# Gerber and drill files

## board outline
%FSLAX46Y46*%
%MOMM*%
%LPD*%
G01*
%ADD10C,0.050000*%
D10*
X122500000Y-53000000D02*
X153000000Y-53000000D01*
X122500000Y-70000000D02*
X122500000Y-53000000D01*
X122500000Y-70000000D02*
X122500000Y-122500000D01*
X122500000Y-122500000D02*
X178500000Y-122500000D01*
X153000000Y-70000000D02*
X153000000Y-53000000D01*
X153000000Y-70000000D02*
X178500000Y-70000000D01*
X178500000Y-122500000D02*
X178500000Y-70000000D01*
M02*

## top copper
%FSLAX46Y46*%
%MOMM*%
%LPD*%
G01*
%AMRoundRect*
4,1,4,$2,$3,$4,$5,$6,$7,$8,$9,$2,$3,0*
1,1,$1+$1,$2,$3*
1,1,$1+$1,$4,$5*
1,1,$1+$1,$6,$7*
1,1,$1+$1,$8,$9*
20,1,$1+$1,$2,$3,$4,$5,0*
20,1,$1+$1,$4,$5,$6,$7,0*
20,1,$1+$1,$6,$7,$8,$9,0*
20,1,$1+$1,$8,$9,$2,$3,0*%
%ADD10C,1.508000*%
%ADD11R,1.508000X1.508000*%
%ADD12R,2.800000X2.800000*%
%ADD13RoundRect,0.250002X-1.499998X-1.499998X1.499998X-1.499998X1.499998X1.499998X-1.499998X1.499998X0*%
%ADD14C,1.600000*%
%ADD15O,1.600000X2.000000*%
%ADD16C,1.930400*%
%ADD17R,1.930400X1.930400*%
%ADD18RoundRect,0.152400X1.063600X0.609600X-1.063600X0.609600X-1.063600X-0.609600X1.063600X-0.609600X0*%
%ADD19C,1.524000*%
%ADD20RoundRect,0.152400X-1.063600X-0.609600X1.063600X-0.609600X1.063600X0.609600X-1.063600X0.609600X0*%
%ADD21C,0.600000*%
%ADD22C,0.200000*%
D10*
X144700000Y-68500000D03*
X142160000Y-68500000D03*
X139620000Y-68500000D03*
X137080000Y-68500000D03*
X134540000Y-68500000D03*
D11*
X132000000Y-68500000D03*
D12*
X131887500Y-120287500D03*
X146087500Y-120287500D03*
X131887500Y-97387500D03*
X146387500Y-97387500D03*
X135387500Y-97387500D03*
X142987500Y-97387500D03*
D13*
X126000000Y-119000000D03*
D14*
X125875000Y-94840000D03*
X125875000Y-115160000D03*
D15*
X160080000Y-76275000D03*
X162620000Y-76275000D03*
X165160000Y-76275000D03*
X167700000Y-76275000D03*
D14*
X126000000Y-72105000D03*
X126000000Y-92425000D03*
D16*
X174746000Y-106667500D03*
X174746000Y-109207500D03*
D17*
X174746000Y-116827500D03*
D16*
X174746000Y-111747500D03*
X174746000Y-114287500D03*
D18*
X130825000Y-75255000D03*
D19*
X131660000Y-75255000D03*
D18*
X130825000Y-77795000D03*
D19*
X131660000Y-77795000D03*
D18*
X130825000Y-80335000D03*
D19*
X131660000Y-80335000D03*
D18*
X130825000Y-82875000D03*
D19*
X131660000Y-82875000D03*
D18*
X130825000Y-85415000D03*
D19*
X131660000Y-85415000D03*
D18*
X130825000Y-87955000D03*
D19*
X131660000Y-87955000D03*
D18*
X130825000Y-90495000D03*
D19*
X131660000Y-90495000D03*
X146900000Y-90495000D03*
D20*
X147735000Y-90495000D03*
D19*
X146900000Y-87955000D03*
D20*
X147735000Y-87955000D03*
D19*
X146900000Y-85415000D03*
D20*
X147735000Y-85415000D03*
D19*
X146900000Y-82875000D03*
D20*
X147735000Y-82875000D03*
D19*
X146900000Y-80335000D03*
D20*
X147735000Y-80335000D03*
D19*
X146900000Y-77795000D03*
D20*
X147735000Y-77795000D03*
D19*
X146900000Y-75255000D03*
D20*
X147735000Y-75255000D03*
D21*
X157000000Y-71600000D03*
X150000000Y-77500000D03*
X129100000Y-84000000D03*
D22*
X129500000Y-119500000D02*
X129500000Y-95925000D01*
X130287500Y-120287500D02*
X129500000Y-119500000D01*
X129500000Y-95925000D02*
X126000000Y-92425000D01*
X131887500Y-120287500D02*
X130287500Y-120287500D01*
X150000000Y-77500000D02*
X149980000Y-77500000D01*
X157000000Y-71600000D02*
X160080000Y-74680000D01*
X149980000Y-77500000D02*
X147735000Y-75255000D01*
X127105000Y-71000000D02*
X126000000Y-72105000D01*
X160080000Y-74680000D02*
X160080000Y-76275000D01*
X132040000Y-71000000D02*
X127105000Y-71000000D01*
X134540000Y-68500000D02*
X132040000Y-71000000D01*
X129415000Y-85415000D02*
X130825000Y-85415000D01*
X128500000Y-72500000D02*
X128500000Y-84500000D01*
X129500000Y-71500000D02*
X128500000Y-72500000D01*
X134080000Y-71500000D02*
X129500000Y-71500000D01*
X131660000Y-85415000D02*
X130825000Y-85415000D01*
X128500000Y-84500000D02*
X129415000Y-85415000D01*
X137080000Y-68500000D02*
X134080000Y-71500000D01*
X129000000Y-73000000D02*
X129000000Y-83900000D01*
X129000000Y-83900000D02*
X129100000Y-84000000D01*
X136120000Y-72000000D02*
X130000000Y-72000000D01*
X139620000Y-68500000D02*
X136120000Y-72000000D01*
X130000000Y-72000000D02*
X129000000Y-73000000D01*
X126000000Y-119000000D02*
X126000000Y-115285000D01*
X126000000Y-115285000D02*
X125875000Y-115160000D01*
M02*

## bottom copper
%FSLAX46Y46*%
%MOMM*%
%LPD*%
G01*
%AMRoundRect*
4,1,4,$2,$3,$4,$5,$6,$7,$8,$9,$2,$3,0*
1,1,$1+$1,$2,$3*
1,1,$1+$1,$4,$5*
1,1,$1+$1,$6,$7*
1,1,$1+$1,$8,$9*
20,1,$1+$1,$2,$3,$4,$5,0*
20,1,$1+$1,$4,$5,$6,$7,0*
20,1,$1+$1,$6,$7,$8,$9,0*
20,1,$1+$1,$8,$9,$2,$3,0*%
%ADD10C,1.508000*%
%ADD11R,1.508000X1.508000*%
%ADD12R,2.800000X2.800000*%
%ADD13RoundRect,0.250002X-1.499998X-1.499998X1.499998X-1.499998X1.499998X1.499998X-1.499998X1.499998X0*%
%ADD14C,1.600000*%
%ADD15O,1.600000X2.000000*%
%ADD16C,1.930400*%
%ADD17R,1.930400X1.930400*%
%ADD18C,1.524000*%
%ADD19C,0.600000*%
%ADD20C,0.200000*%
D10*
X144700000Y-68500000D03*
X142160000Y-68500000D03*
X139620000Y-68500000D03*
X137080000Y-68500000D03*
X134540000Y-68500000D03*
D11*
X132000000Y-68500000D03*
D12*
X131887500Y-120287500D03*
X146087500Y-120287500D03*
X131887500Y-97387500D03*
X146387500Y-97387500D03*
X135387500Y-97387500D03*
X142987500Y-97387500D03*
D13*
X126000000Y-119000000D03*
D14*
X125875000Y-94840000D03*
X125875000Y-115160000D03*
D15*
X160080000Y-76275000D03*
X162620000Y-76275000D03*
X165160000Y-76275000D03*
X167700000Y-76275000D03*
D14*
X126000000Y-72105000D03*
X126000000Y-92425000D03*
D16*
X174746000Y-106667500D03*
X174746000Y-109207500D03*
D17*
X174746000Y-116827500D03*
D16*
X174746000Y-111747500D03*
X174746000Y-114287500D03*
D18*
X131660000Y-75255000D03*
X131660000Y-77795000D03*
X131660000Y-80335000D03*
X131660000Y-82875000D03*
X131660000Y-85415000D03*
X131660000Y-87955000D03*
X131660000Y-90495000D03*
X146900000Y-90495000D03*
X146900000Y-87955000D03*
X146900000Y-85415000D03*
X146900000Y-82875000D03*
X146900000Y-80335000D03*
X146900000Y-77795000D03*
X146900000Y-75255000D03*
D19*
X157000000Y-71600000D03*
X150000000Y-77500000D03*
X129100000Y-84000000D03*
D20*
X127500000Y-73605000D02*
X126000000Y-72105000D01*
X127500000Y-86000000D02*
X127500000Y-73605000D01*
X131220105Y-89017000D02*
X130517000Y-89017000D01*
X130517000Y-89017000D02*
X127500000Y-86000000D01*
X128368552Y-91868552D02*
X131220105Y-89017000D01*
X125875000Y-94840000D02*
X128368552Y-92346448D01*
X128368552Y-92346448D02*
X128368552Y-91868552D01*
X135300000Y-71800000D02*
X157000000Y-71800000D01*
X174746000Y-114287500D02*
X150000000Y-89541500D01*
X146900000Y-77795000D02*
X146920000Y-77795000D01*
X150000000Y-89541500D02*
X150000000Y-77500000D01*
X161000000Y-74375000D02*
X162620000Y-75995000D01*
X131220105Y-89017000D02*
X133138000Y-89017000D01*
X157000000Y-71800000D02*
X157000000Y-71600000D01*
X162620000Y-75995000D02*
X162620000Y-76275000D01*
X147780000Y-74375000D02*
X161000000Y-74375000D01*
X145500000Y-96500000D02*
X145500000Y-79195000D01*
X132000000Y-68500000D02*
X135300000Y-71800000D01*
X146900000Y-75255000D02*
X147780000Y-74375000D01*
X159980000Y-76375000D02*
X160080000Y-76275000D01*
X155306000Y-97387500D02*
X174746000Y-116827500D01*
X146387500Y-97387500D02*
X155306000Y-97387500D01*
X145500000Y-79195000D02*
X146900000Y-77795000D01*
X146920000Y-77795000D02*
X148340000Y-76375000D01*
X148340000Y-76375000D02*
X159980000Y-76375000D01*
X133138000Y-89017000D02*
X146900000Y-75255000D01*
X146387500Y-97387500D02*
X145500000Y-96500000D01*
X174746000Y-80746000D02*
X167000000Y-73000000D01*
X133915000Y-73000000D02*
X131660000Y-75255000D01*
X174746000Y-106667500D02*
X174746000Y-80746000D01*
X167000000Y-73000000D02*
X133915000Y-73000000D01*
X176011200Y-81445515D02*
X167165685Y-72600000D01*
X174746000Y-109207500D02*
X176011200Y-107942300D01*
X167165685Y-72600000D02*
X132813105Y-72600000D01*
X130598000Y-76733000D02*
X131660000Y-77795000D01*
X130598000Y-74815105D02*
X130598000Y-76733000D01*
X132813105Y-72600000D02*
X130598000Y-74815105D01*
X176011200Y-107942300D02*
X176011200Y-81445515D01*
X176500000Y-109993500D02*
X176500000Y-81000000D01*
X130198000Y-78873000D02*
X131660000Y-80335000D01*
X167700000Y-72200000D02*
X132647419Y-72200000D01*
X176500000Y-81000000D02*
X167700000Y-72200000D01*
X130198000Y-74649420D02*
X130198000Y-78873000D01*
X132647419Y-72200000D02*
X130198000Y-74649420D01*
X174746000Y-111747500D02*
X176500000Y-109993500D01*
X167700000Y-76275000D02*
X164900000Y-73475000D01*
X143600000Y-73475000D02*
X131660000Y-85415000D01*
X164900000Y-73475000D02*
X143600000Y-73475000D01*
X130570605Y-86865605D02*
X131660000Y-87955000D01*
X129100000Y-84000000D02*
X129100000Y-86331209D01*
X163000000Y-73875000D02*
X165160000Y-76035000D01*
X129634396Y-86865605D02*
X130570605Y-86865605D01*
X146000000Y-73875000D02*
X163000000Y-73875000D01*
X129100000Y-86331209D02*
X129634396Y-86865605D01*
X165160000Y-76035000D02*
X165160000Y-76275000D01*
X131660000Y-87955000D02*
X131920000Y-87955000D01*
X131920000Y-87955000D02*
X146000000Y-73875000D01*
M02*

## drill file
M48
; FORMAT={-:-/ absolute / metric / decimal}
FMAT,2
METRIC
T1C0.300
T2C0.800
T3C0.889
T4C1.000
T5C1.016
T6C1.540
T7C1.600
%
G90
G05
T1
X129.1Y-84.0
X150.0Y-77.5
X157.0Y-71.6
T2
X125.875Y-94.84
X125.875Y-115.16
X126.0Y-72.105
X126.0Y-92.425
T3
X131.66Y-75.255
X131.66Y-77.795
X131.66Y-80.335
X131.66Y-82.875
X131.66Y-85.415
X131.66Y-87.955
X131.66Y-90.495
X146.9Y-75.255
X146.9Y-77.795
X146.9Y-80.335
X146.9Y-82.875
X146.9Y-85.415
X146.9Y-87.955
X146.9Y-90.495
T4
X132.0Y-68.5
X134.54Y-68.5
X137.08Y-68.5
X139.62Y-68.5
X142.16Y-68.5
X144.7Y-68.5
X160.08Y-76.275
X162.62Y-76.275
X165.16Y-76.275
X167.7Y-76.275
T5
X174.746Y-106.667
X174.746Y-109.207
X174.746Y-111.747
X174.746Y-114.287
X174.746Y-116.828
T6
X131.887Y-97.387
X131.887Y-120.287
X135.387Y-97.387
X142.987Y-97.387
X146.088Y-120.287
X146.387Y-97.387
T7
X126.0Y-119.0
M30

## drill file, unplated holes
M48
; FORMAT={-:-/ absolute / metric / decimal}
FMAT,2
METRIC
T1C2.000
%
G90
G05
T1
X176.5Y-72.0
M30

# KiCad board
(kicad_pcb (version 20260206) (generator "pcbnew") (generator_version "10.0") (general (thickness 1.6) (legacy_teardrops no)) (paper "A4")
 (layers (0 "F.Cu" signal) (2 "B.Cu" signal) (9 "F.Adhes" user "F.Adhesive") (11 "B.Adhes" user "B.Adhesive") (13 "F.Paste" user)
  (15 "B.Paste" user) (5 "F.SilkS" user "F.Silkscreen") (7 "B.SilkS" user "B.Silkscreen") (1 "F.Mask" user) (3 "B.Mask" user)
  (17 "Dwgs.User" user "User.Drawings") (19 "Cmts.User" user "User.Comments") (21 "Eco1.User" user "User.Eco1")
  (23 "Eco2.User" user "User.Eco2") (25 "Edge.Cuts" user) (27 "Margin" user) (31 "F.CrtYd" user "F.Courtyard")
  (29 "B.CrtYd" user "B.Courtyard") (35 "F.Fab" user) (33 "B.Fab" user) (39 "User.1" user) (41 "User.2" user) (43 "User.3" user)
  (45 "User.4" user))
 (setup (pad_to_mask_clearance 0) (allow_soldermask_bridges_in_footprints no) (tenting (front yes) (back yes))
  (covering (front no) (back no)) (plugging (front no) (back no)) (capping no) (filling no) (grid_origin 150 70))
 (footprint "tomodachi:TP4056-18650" (layer "F.Cu") (at 130.1875 121.9875 90)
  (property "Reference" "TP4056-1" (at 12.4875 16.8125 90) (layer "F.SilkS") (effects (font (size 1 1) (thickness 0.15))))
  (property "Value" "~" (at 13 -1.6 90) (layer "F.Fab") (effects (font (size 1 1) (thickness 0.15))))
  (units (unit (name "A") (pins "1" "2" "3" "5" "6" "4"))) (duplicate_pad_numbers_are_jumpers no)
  (pad "1" thru_hole rect (at 1.7 1.7 90) (size 2.8 2.8) (drill 1.54) (layers "*.Cu" "*.Mask") (remove_unused_layers no) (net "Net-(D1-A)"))
  (pad "2" thru_hole rect (at 1.7 15.9 90) (size 2.8 2.8) (drill 1.54) (layers "*.Cu" "*.Mask") (remove_unused_layers no) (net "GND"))
  (pad "3" thru_hole rect (at 24.6 1.7 90) (size 2.8 2.8) (drill 1.54) (layers "*.Cu" "*.Mask") (remove_unused_layers no)
   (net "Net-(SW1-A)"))
  (pad "4" thru_hole rect (at 24.6 16.2 90) (size 2.8 2.8) (drill 1.54) (layers "*.Cu" "*.Mask") (remove_unused_layers no)
   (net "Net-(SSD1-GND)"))
  (pad "5" thru_hole rect (at 24.6 5.2 90) (size 2.8 2.8) (drill 1.54) (layers "*.Cu" "*.Mask") (remove_unused_layers no)
   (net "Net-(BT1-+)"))
  (pad "6" thru_hole rect (at 24.6 12.8 90) (size 2.8 2.8) (drill 1.54) (layers "*.Cu" "*.Mask") (remove_unused_layers no)
   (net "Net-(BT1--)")))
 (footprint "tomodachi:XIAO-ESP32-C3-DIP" (layer "F.Cu") (at 139.28 82.875 90)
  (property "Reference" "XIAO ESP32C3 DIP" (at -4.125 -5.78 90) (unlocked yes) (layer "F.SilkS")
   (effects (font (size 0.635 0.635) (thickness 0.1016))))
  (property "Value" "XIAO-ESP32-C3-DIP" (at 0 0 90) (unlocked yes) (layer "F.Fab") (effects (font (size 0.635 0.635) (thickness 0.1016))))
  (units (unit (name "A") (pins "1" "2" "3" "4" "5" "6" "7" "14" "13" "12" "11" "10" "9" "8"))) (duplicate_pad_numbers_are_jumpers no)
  (pad "1" smd roundrect (at 7.62 -8.455 180) (size 2.432 1.524) (layers "F.Cu" "F.Mask") (roundrect_rratio 0.1)
   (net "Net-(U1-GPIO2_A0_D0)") (thermal_bridge_angle 45))
  (pad "1" thru_hole circle (at 7.62 -7.62 180) (size 1.524 1.524) (drill 0.889) (layers "*.Cu" "*.Mask") (remove_unused_layers no)
   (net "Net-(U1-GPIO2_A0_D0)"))
  (pad "2" smd roundrect (at 5.08 -8.455 180) (size 2.432 1.524) (layers "F.Cu" "F.Mask") (roundrect_rratio 0.1)
   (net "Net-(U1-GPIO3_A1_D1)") (thermal_bridge_angle 45))
  (pad "2" thru_hole circle (at 5.08 -7.62 180) (size 1.524 1.524) (drill 0.889) (layers "*.Cu" "*.Mask") (remove_unused_layers no)
   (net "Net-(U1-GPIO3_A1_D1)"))
  (pad "3" smd roundrect (at 2.54 -8.455 180) (size 2.432 1.524) (layers "F.Cu" "F.Mask") (roundrect_rratio 0.1)
   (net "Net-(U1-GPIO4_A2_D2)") (thermal_bridge_angle 45))
  (pad "3" thru_hole circle (at 2.54 -7.62 180) (size 1.524 1.524) (drill 0.889) (layers "*.Cu" "*.Mask") (remove_unused_layers no)
   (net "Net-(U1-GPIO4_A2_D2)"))
  (pad "4" smd roundrect (at 0 -8.455 180) (size 2.432 1.524) (layers "F.Cu" "F.Mask") (roundrect_rratio 0.1)
   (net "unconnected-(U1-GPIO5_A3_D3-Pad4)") (thermal_bridge_angle 45))
  (pad "4" thru_hole circle (at 0 -7.62 180) (size 1.524 1.524) (drill 0.889) (layers "*.Cu" "*.Mask") (remove_unused_layers no)
   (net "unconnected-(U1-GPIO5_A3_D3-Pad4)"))
  (pad "5" smd roundrect (at -2.54 -8.455 180) (size 2.432 1.524) (layers "F.Cu" "F.Mask") (roundrect_rratio 0.1) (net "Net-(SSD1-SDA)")
   (thermal_bridge_angle 45))
  (pad "5" thru_hole circle (at -2.54 -7.62 180) (size 1.524 1.524) (drill 0.889) (layers "*.Cu" "*.Mask") (remove_unused_layers no)
   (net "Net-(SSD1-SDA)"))
  (pad "6" smd roundrect (at -5.08 -8.455 180) (size 2.432 1.524) (layers "F.Cu" "F.Mask") (roundrect_rratio 0.1) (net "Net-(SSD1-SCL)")
   (thermal_bridge_angle 45))
  (pad "6" thru_hole circle (at -5.08 -7.62 180) (size 1.524 1.524) (drill 0.889) (layers "*.Cu" "*.Mask") (remove_unused_layers no)
   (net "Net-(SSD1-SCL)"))
  (pad "7" smd roundrect (at -7.62 -8.455 180) (size 2.432 1.524) (layers "F.Cu" "F.Mask") (roundrect_rratio 0.1)
   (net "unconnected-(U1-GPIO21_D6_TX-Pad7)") (thermal_bridge_angle 45))
  (pad "7" thru_hole circle (at -7.62 -7.62 180) (size 1.524 1.524) (drill 0.889) (layers "*.Cu" "*.Mask") (remove_unused_layers no)
   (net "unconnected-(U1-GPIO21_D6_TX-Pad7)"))
  (pad "8" thru_hole circle (at -7.62 7.62) (size 1.524 1.524) (drill 0.889) (layers "*.Cu" "*.Mask") (remove_unused_layers no)
   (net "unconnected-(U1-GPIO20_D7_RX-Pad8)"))
  (pad "8" smd roundrect (at -7.62 8.455) (size 2.432 1.524) (layers "F.Cu" "F.Mask") (roundrect_rratio 0.1)
   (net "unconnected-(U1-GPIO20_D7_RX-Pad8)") (thermal_bridge_angle 45))
  (pad "9" thru_hole circle (at -5.08 7.62) (size 1.524 1.524) (drill 0.889) (layers "*.Cu" "*.Mask") (remove_unused_layers no)
   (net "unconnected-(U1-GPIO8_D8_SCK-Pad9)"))
  (pad "9" smd roundrect (at -5.08 8.455) (size 2.432 1.524) (layers "F.Cu" "F.Mask") (roundrect_rratio 0.1)
   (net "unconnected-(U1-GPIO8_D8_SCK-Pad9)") (thermal_bridge_angle 45))
  (pad "10" thru_hole circle (at -2.54 7.62) (size 1.524 1.524) (drill 0.889) (layers "*.Cu" "*.Mask") (remove_unused_layers no)
   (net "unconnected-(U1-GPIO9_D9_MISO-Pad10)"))
  (pad "10" smd roundrect (at -2.54 8.455) (size 2.432 1.524) (layers "F.Cu" "F.Mask") (roundrect_rratio 0.1)
   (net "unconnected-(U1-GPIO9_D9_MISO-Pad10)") (thermal_bridge_angle 45))
  (pad "11" thru_hole circle (at 0 7.62) (size 1.524 1.524) (drill 0.889) (layers "*.Cu" "*.Mask") (remove_unused_layers no)
   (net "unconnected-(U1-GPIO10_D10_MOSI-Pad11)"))
  (pad "11" smd roundrect (at 0 8.455) (size 2.432 1.524) (layers "F.Cu" "F.Mask") (roundrect_rratio 0.1)
   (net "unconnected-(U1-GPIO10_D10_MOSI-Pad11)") (thermal_bridge_angle 45))
  (pad "12" thru_hole circle (at 2.54 7.62) (size 1.524 1.524) (drill 0.889) (layers "*.Cu" "*.Mask") (remove_unused_layers no)
   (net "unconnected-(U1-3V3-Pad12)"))
  (pad "12" smd roundrect (at 2.54 8.455) (size 2.432 1.524) (layers "F.Cu" "F.Mask") (roundrect_rratio 0.1)
   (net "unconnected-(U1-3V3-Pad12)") (thermal_bridge_angle 45))
  (pad "13" thru_hole circle (at 5.08 7.62) (size 1.524 1.524) (drill 0.889) (layers "*.Cu" "*.Mask") (remove_unused_layers no)
   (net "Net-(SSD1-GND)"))
  (pad "13" smd roundrect (at 5.08 8.455) (size 2.432 1.524) (layers "F.Cu" "F.Mask") (roundrect_rratio 0.1) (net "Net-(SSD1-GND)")
   (thermal_bridge_angle 45))
  (pad "14" thru_hole circle (at 7.62 7.62) (size 1.524 1.524) (drill 0.889) (layers "*.Cu" "*.Mask") (remove_unused_layers no)
   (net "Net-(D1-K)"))
  (pad "14" smd roundrect (at 7.62 8.455) (size 2.432 1.524) (layers "F.Cu" "F.Mask") (roundrect_rratio 0.1) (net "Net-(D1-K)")
   (thermal_bridge_angle 45)))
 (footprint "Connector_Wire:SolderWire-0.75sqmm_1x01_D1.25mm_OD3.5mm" (layer "F.Cu") (at 126 119)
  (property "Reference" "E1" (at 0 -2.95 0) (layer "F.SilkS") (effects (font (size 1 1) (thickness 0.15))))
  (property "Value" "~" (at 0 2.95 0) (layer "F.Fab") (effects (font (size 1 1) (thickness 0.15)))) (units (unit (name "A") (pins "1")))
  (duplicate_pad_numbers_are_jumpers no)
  (pad "1" thru_hole roundrect (at 0 0) (size 3.5 3.5) (drill 1.6) (layers "*.Cu" "*.Mask") (remove_unused_layers no)
   (roundrect_rratio 0.071429) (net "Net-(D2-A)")))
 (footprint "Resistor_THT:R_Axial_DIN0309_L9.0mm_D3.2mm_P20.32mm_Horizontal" (layer "F.Cu") (at 125.875 94.84 -90)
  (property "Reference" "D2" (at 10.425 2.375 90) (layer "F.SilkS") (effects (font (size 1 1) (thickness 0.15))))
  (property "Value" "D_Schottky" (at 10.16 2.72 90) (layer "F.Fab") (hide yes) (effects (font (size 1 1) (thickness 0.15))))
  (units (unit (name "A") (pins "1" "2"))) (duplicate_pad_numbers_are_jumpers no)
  (pad "1" thru_hole circle (at 0 0 270) (size 1.6 1.6) (drill 0.8) (layers "*.Cu" "*.Mask") (remove_unused_layers no) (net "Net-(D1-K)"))
  (pad "2" thru_hole circle (at 20.32 0 270) (size 1.6 1.6) (drill 0.8) (layers "*.Cu" "*.Mask") (remove_unused_layers no)
   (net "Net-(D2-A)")))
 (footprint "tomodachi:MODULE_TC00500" (layer "F.Cu") (at 138.35 68.5 90)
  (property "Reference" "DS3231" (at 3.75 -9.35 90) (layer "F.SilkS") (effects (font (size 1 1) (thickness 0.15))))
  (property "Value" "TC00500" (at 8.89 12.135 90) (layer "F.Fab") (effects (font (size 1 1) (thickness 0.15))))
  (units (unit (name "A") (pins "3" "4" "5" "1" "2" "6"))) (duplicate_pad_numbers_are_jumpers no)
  (pad "1" thru_hole circle (at 0 6.35 90) (size 1.508 1.508) (drill 1) (layers "*.Cu" "*.Mask") (remove_unused_layers no)
   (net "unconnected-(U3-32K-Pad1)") (solder_mask_margin 0.102))
  (pad "2" thru_hole circle (at 0 3.81 90) (size 1.508 1.508) (drill 1) (layers "*.Cu" "*.Mask") (remove_unused_layers no)
   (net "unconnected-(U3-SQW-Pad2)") (solder_mask_margin 0.102))
  (pad "3" thru_hole circle (at 0 1.27 90) (size 1.508 1.508) (drill 1) (layers "*.Cu" "*.Mask") (remove_unused_layers no)
   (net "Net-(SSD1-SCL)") (solder_mask_margin 0.102))
  (pad "4" thru_hole circle (at 0 -1.27 90) (size 1.508 1.508) (drill 1) (layers "*.Cu" "*.Mask") (remove_unused_layers no)
   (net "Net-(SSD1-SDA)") (solder_mask_margin 0.102))
  (pad "5" thru_hole circle (at 0 -3.81 90) (size 1.508 1.508) (drill 1) (layers "*.Cu" "*.Mask") (remove_unused_layers no)
   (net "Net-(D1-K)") (solder_mask_margin 0.102))
  (pad "6" thru_hole rect (at 0 -6.35 90) (size 1.508 1.508) (drill 1) (layers "*.Cu" "*.Mask") (remove_unused_layers no)
   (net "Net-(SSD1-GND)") (solder_mask_margin 0.102)))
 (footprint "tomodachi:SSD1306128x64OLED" (layer "F.Cu") (at 163.7 86.875)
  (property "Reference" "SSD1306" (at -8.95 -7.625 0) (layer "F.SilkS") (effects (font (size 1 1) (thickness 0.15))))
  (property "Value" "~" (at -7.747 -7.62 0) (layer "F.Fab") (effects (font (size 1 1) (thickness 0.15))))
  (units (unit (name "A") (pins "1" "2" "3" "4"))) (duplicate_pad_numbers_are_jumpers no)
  (pad "1" thru_hole oval (at -3.62 -10.6 90) (size 2 1.6) (drill 1) (layers "*.Cu" "*.Mask") (remove_unused_layers no)
   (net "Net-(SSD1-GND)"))
  (pad "2" thru_hole oval (at -1.08 -10.6 90) (size 2 1.6) (drill 1) (layers "*.Cu" "*.Mask") (remove_unused_layers no) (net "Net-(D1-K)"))
  (pad "3" thru_hole oval (at 1.46 -10.6 90) (size 2 1.6) (drill 1) (layers "*.Cu" "*.Mask") (remove_unused_layers no)
   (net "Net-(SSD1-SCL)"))
  (pad "4" thru_hole oval (at 4 -10.6 90) (size 2 1.6) (drill 1) (layers "*.Cu" "*.Mask") (remove_unused_layers no) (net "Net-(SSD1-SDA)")))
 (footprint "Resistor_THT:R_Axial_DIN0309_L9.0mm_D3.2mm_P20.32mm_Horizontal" (layer "F.Cu") (at 126 72.105 -90)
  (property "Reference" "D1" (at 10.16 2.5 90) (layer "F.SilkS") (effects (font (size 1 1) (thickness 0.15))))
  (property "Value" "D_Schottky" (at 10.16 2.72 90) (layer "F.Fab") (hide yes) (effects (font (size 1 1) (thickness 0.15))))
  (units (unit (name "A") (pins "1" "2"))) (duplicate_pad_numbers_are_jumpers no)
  (pad "1" thru_hole circle (at 0 0 270) (size 1.6 1.6) (drill 0.8) (layers "*.Cu" "*.Mask") (remove_unused_layers no) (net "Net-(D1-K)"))
  (pad "2" thru_hole circle (at 20.32 0 270) (size 1.6 1.6) (drill 0.8) (layers "*.Cu" "*.Mask") (remove_unused_layers no)
   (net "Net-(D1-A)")))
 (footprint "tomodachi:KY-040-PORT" (layer "F.Cu") (at 164 111.875 -90)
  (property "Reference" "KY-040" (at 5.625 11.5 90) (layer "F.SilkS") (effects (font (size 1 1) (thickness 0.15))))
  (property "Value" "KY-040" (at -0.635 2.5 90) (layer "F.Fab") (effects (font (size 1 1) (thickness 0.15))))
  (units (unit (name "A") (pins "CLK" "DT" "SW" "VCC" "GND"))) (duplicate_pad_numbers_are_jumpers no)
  (pad "CLK" thru_hole circle (at -5.2075 -10.746 270) (size 1.9304 1.9304) (drill 1.016) (layers "*.Cu" "*.Mask") (remove_unused_layers no)
   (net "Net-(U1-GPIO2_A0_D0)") (solder_mask_margin 0.102))
  (pad "DT" thru_hole circle (at -2.6675 -10.746 270) (size 1.9304 1.9304) (drill 1.016) (layers "*.Cu" "*.Mask") (remove_unused_layers no)
   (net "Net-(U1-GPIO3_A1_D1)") (solder_mask_margin 0.102))
  (pad "GND" thru_hole rect (at 4.9525 -10.746 270) (size 1.9304 1.9304) (drill 1.016) (layers "*.Cu" "*.Mask") (remove_unused_layers no)
   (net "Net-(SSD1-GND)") (solder_mask_margin 0.102))
  (pad "SW" thru_hole circle (at -0.1275 -10.746 270) (size 1.9304 1.9304) (drill 1.016) (layers "*.Cu" "*.Mask") (remove_unused_layers no)
   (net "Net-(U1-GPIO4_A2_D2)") (solder_mask_margin 0.102))
  (pad "VCC" thru_hole circle (at 2.4125 -10.746 270) (size 1.9304 1.9304) (drill 1.016) (layers "*.Cu" "*.Mask") (remove_unused_layers no)
   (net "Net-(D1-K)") (solder_mask_margin 0.102)))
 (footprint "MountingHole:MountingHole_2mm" (layer "F.Cu") (at 176.5 72)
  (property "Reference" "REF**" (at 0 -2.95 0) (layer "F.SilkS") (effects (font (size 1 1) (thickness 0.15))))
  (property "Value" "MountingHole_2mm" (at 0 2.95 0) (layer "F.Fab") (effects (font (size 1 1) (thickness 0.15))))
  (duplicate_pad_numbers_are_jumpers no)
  (pad "" np_thru_hole circle (at 0 0) (size 2 2) (drill 2) (layers "*.Cu" "*.Mask")))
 (gr_line (start 122.5 53) (end 153 53) (stroke (width 0.05) (type default)) (layer "Edge.Cuts"))
 (gr_line (start 122.5 70) (end 122.5 53) (stroke (width 0.05) (type default)) (layer "Edge.Cuts"))
 (gr_line (start 122.5 70) (end 122.5 122.5) (stroke (width 0.05) (type default)) (layer "Edge.Cuts"))
 (gr_line (start 122.5 122.5) (end 178.5 122.5) (stroke (width 0.05) (type default)) (layer "Edge.Cuts"))
 (gr_line (start 153 70) (end 153 53) (stroke (width 0.05) (type default)) (layer "Edge.Cuts"))
 (gr_line (start 153 70) (end 178.5 70) (stroke (width 0.05) (type default)) (layer "Edge.Cuts"))
 (gr_line (start 178.5 122.5) (end 178.5 70) (stroke (width 0.05) (type default)) (layer "Edge.Cuts"))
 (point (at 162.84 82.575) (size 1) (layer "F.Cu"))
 (segment (start 129.5 119.5) (end 129.5 95.925) (width 0.2) (layer "F.Cu") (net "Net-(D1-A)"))
 (segment (start 129.5 95.925) (end 126 92.425) (width 0.2) (layer "F.Cu") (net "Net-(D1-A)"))
 (segment (start 131.8875 120.2875) (end 130.2875 120.2875) (width 0.2) (layer "F.Cu") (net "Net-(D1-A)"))
 (segment (start 130.2875 120.2875) (end 129.5 119.5) (width 0.2) (layer "F.Cu") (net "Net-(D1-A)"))
 (segment (start 150 77.5) (end 149.98 77.5) (width 0.2) (layer "F.Cu") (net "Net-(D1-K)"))
 (segment (start 149.98 77.5) (end 147.735 75.255) (width 0.2) (layer "F.Cu") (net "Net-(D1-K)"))
 (segment (start 127.105 71) (end 126 72.105) (width 0.2) (layer "F.Cu") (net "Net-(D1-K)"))
 (segment (start 132.04 71) (end 127.105 71) (width 0.2) (layer "F.Cu") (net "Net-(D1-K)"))
 (segment (start 134.54 68.5) (end 132.04 71) (width 0.2) (layer "F.Cu") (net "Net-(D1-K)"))
 (via (at 150 77.5) (size 0.6) (drill 0.3) (layers "F.Cu" "B.Cu") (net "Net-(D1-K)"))
 (segment (start 174.746 114.2875) (end 150 89.5415) (width 0.2) (layer "B.Cu") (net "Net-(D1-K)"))
 (segment (start 150 89.5415) (end 150 77.5) (width 0.2) (layer "B.Cu") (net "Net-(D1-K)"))
 (segment (start 161 74.375) (end 162.62 75.995) (width 0.2) (layer "B.Cu") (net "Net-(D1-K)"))
 (segment (start 131.220105 89.017) (end 133.138 89.017) (width 0.2) (layer "B.Cu") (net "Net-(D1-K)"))
 (segment (start 131.220105 89.017) (end 130.517 89.017) (width 0.2) (layer "B.Cu") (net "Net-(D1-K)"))
 (segment (start 162.62 75.995) (end 162.62 76.275) (width 0.2) (layer "B.Cu") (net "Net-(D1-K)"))
 (segment (start 147.78 74.375) (end 161 74.375) (width 0.2) (layer "B.Cu") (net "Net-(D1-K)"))
 (segment (start 127.5 86) (end 127.5 73.605) (width 0.2) (layer "B.Cu") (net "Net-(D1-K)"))
 (segment (start 130.517 89.017) (end 127.5 86) (width 0.2) (layer "B.Cu") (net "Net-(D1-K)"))
 (segment (start 127.5 73.605) (end 126 72.105) (width 0.2) (layer "B.Cu") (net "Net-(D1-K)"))
 (segment (start 125.875 94.84) (end 128.368552 92.346448) (width 0.2) (layer "B.Cu") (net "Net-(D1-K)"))
 (segment (start 128.368552 91.868552) (end 131.220105 89.017) (width 0.2) (layer "B.Cu") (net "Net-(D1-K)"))
 (segment (start 146.9 75.255) (end 147.78 74.375) (width 0.2) (layer "B.Cu") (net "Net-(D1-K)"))
 (segment (start 128.368552 92.346448) (end 128.368552 91.868552) (width 0.2) (layer "B.Cu") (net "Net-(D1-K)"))
 (segment (start 133.138 89.017) (end 146.9 75.255) (width 0.2) (layer "B.Cu") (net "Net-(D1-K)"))
 (segment (start 174.746 80.746) (end 167 73) (width 0.2) (layer "B.Cu") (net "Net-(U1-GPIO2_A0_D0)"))
 (segment (start 133.915 73) (end 131.66 75.255) (width 0.2) (layer "B.Cu") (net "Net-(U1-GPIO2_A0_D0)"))
 (segment (start 174.746 106.6675) (end 174.746 80.746) (width 0.2) (layer "B.Cu") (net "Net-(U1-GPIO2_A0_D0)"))
 (segment (start 167 73) (end 133.915 73) (width 0.2) (layer "B.Cu") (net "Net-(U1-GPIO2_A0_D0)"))
 (segment (start 176.0112 81.445515) (end 167.165685 72.6) (width 0.2) (layer "B.Cu") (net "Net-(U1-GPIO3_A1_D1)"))
 (segment (start 174.746 109.2075) (end 176.0112 107.9423) (width 0.2) (layer "B.Cu") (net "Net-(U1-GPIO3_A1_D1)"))
 (segment (start 167.165685 72.6) (end 132.813105 72.6) (width 0.2) (layer "B.Cu") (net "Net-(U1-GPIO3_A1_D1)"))
 (segment (start 130.598 76.733) (end 131.66 77.795) (width 0.2) (layer "B.Cu") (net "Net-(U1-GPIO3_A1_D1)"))
 (segment (start 130.598 74.815105) (end 130.598 76.733) (width 0.2) (layer "B.Cu") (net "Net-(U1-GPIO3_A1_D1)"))
 (segment (start 132.813105 72.6) (end 130.598 74.815105) (width 0.2) (layer "B.Cu") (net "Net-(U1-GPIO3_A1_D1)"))
 (segment (start 176.0112 107.9423) (end 176.0112 81.445515) (width 0.2) (layer "B.Cu") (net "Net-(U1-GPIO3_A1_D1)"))
 (segment (start 176.5 109.9935) (end 176.5 81) (width 0.2) (layer "B.Cu") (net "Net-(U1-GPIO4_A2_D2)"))
 (segment (start 130.198 78.873) (end 131.66 80.335) (width 0.2) (layer "B.Cu") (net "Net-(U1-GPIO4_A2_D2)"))
 (segment (start 167.7 72.2) (end 132.647419 72.2) (width 0.2) (layer "B.Cu") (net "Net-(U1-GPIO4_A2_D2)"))
 (segment (start 176.5 81) (end 167.7 72.2) (width 0.2) (layer "B.Cu") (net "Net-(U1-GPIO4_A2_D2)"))
 (segment (start 130.198 74.64942) (end 130.198 78.873) (width 0.2) (layer "B.Cu") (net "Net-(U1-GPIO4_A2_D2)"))
 (segment (start 132.647419 72.2) (end 130.198 74.64942) (width 0.2) (layer "B.Cu") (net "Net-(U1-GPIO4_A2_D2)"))
 (segment (start 174.746 111.7475) (end 176.5 109.9935) (width 0.2) (layer "B.Cu") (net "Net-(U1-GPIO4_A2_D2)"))
 (segment (start 129.415 85.415) (end 130.825 85.415) (width 0.2) (layer "F.Cu") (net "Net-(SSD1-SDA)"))
 (segment (start 128.5 72.5) (end 128.5 84.5) (width 0.2) (layer "F.Cu") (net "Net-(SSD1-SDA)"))
 (segment (start 129.5 71.5) (end 128.5 72.5) (width 0.2) (layer "F.Cu") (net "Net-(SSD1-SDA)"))
 (segment (start 134.08 71.5) (end 129.5 71.5) (width 0.2) (layer "F.Cu") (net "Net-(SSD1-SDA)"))
 (segment (start 131.66 85.415) (end 130.825 85.415) (width 0.2) (layer "F.Cu") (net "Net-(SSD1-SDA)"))
 (segment (start 128.5 84.5) (end 129.415 85.415) (width 0.2) (layer "F.Cu") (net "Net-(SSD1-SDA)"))
 (segment (start 137.08 68.5) (end 134.08 71.5) (width 0.2) (layer "F.Cu") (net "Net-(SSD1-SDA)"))
 (segment (start 167.7 76.275) (end 164.9 73.475) (width 0.2) (layer "B.Cu") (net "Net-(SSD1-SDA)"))
 (segment (start 143.6 73.475) (end 131.66 85.415) (width 0.2) (layer "B.Cu") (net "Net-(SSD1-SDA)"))
 (segment (start 164.9 73.475) (end 143.6 73.475) (width 0.2) (layer "B.Cu") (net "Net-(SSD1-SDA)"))
 (segment (start 129 73) (end 129 83.9) (width 0.2) (layer "F.Cu") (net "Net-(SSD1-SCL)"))
 (segment (start 129 83.9) (end 129.1 84) (width 0.2) (layer "F.Cu") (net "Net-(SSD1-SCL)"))
 (segment (start 136.12 72) (end 130 72) (width 0.2) (layer "F.Cu") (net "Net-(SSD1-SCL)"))
 (segment (start 139.62 68.5) (end 136.12 72) (width 0.2) (layer "F.Cu") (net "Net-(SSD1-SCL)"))
 (segment (start 130 72) (end 129 73) (width 0.2) (layer "F.Cu") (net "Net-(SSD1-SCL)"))
 (via (at 129.1 84) (size 0.6) (drill 0.3) (layers "F.Cu" "B.Cu") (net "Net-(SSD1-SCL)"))
 (segment (start 130.570605 86.865605) (end 131.66 87.955) (width 0.2) (layer "B.Cu") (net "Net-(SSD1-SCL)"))
 (segment (start 129.1 84) (end 129.1 86.331209) (width 0.2) (layer "B.Cu") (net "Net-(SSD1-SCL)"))
 (segment (start 163 73.875) (end 165.16 76.035) (width 0.2) (layer "B.Cu") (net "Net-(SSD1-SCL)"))
 (segment (start 129.634396 86.865605) (end 130.570605 86.865605) (width 0.2) (layer "B.Cu") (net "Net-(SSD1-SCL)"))
 (segment (start 146 73.875) (end 163 73.875) (width 0.2) (layer "B.Cu") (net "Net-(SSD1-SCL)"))
 (segment (start 129.1 86.331209) (end 129.634396 86.865605) (width 0.2) (layer "B.Cu") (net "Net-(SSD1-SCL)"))
 (segment (start 165.16 76.035) (end 165.16 76.275) (width 0.2) (layer "B.Cu") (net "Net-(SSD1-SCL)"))
 (segment (start 131.66 87.955) (end 131.92 87.955) (width 0.2) (layer "B.Cu") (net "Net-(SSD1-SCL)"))
 (segment (start 131.92 87.955) (end 146 73.875) (width 0.2) (layer "B.Cu") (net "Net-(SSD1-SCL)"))
 (segment (start 126 119) (end 126 115.285) (width 0.2) (layer "F.Cu") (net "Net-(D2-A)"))
 (segment (start 126 115.285) (end 125.875 115.16) (width 0.2) (layer "F.Cu") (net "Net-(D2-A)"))
 (segment (start 157 71.6) (end 160.08 74.68) (width 0.2) (layer "F.Cu") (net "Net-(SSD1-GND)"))
 (segment (start 160.08 74.68) (end 160.08 76.275) (width 0.2) (layer "F.Cu") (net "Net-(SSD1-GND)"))
 (via (at 157 71.6) (size 0.6) (drill 0.3) (layers "F.Cu" "B.Cu") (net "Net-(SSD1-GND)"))
 (segment (start 135.3 71.8) (end 157 71.8) (width 0.2) (layer "B.Cu") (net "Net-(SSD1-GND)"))
 (segment (start 146.9 77.795) (end 146.92 77.795) (width 0.2) (layer "B.Cu") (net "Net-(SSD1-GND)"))
 (segment (start 157 71.8) (end 157 71.6) (width 0.2) (layer "B.Cu") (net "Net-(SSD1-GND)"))
 (segment (start 145.5 96.5) (end 145.5 79.195) (width 0.2) (layer "B.Cu") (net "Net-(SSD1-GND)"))
 (segment (start 132 68.5) (end 135.3 71.8) (width 0.2) (layer "B.Cu") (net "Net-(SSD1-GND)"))
 (segment (start 159.98 76.375) (end 160.08 76.275) (width 0.2) (layer "B.Cu") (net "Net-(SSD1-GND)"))
 (segment (start 155.306 97.3875) (end 174.746 116.8275) (width 0.2) (layer "B.Cu") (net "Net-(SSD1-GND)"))
 (segment (start 146.3875 97.3875) (end 155.306 97.3875) (width 0.2) (layer "B.Cu") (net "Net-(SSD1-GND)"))
 (segment (start 145.5 79.195) (end 146.9 77.795) (width 0.2) (layer "B.Cu") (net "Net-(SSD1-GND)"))
 (segment (start 146.92 77.795) (end 148.34 76.375) (width 0.2) (layer "B.Cu") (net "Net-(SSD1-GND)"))
 (segment (start 148.34 76.375) (end 159.98 76.375) (width 0.2) (layer "B.Cu") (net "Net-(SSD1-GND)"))
 (segment (start 146.3875 97.3875) (end 145.5 96.5) (width 0.2) (layer "B.Cu") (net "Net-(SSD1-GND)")))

